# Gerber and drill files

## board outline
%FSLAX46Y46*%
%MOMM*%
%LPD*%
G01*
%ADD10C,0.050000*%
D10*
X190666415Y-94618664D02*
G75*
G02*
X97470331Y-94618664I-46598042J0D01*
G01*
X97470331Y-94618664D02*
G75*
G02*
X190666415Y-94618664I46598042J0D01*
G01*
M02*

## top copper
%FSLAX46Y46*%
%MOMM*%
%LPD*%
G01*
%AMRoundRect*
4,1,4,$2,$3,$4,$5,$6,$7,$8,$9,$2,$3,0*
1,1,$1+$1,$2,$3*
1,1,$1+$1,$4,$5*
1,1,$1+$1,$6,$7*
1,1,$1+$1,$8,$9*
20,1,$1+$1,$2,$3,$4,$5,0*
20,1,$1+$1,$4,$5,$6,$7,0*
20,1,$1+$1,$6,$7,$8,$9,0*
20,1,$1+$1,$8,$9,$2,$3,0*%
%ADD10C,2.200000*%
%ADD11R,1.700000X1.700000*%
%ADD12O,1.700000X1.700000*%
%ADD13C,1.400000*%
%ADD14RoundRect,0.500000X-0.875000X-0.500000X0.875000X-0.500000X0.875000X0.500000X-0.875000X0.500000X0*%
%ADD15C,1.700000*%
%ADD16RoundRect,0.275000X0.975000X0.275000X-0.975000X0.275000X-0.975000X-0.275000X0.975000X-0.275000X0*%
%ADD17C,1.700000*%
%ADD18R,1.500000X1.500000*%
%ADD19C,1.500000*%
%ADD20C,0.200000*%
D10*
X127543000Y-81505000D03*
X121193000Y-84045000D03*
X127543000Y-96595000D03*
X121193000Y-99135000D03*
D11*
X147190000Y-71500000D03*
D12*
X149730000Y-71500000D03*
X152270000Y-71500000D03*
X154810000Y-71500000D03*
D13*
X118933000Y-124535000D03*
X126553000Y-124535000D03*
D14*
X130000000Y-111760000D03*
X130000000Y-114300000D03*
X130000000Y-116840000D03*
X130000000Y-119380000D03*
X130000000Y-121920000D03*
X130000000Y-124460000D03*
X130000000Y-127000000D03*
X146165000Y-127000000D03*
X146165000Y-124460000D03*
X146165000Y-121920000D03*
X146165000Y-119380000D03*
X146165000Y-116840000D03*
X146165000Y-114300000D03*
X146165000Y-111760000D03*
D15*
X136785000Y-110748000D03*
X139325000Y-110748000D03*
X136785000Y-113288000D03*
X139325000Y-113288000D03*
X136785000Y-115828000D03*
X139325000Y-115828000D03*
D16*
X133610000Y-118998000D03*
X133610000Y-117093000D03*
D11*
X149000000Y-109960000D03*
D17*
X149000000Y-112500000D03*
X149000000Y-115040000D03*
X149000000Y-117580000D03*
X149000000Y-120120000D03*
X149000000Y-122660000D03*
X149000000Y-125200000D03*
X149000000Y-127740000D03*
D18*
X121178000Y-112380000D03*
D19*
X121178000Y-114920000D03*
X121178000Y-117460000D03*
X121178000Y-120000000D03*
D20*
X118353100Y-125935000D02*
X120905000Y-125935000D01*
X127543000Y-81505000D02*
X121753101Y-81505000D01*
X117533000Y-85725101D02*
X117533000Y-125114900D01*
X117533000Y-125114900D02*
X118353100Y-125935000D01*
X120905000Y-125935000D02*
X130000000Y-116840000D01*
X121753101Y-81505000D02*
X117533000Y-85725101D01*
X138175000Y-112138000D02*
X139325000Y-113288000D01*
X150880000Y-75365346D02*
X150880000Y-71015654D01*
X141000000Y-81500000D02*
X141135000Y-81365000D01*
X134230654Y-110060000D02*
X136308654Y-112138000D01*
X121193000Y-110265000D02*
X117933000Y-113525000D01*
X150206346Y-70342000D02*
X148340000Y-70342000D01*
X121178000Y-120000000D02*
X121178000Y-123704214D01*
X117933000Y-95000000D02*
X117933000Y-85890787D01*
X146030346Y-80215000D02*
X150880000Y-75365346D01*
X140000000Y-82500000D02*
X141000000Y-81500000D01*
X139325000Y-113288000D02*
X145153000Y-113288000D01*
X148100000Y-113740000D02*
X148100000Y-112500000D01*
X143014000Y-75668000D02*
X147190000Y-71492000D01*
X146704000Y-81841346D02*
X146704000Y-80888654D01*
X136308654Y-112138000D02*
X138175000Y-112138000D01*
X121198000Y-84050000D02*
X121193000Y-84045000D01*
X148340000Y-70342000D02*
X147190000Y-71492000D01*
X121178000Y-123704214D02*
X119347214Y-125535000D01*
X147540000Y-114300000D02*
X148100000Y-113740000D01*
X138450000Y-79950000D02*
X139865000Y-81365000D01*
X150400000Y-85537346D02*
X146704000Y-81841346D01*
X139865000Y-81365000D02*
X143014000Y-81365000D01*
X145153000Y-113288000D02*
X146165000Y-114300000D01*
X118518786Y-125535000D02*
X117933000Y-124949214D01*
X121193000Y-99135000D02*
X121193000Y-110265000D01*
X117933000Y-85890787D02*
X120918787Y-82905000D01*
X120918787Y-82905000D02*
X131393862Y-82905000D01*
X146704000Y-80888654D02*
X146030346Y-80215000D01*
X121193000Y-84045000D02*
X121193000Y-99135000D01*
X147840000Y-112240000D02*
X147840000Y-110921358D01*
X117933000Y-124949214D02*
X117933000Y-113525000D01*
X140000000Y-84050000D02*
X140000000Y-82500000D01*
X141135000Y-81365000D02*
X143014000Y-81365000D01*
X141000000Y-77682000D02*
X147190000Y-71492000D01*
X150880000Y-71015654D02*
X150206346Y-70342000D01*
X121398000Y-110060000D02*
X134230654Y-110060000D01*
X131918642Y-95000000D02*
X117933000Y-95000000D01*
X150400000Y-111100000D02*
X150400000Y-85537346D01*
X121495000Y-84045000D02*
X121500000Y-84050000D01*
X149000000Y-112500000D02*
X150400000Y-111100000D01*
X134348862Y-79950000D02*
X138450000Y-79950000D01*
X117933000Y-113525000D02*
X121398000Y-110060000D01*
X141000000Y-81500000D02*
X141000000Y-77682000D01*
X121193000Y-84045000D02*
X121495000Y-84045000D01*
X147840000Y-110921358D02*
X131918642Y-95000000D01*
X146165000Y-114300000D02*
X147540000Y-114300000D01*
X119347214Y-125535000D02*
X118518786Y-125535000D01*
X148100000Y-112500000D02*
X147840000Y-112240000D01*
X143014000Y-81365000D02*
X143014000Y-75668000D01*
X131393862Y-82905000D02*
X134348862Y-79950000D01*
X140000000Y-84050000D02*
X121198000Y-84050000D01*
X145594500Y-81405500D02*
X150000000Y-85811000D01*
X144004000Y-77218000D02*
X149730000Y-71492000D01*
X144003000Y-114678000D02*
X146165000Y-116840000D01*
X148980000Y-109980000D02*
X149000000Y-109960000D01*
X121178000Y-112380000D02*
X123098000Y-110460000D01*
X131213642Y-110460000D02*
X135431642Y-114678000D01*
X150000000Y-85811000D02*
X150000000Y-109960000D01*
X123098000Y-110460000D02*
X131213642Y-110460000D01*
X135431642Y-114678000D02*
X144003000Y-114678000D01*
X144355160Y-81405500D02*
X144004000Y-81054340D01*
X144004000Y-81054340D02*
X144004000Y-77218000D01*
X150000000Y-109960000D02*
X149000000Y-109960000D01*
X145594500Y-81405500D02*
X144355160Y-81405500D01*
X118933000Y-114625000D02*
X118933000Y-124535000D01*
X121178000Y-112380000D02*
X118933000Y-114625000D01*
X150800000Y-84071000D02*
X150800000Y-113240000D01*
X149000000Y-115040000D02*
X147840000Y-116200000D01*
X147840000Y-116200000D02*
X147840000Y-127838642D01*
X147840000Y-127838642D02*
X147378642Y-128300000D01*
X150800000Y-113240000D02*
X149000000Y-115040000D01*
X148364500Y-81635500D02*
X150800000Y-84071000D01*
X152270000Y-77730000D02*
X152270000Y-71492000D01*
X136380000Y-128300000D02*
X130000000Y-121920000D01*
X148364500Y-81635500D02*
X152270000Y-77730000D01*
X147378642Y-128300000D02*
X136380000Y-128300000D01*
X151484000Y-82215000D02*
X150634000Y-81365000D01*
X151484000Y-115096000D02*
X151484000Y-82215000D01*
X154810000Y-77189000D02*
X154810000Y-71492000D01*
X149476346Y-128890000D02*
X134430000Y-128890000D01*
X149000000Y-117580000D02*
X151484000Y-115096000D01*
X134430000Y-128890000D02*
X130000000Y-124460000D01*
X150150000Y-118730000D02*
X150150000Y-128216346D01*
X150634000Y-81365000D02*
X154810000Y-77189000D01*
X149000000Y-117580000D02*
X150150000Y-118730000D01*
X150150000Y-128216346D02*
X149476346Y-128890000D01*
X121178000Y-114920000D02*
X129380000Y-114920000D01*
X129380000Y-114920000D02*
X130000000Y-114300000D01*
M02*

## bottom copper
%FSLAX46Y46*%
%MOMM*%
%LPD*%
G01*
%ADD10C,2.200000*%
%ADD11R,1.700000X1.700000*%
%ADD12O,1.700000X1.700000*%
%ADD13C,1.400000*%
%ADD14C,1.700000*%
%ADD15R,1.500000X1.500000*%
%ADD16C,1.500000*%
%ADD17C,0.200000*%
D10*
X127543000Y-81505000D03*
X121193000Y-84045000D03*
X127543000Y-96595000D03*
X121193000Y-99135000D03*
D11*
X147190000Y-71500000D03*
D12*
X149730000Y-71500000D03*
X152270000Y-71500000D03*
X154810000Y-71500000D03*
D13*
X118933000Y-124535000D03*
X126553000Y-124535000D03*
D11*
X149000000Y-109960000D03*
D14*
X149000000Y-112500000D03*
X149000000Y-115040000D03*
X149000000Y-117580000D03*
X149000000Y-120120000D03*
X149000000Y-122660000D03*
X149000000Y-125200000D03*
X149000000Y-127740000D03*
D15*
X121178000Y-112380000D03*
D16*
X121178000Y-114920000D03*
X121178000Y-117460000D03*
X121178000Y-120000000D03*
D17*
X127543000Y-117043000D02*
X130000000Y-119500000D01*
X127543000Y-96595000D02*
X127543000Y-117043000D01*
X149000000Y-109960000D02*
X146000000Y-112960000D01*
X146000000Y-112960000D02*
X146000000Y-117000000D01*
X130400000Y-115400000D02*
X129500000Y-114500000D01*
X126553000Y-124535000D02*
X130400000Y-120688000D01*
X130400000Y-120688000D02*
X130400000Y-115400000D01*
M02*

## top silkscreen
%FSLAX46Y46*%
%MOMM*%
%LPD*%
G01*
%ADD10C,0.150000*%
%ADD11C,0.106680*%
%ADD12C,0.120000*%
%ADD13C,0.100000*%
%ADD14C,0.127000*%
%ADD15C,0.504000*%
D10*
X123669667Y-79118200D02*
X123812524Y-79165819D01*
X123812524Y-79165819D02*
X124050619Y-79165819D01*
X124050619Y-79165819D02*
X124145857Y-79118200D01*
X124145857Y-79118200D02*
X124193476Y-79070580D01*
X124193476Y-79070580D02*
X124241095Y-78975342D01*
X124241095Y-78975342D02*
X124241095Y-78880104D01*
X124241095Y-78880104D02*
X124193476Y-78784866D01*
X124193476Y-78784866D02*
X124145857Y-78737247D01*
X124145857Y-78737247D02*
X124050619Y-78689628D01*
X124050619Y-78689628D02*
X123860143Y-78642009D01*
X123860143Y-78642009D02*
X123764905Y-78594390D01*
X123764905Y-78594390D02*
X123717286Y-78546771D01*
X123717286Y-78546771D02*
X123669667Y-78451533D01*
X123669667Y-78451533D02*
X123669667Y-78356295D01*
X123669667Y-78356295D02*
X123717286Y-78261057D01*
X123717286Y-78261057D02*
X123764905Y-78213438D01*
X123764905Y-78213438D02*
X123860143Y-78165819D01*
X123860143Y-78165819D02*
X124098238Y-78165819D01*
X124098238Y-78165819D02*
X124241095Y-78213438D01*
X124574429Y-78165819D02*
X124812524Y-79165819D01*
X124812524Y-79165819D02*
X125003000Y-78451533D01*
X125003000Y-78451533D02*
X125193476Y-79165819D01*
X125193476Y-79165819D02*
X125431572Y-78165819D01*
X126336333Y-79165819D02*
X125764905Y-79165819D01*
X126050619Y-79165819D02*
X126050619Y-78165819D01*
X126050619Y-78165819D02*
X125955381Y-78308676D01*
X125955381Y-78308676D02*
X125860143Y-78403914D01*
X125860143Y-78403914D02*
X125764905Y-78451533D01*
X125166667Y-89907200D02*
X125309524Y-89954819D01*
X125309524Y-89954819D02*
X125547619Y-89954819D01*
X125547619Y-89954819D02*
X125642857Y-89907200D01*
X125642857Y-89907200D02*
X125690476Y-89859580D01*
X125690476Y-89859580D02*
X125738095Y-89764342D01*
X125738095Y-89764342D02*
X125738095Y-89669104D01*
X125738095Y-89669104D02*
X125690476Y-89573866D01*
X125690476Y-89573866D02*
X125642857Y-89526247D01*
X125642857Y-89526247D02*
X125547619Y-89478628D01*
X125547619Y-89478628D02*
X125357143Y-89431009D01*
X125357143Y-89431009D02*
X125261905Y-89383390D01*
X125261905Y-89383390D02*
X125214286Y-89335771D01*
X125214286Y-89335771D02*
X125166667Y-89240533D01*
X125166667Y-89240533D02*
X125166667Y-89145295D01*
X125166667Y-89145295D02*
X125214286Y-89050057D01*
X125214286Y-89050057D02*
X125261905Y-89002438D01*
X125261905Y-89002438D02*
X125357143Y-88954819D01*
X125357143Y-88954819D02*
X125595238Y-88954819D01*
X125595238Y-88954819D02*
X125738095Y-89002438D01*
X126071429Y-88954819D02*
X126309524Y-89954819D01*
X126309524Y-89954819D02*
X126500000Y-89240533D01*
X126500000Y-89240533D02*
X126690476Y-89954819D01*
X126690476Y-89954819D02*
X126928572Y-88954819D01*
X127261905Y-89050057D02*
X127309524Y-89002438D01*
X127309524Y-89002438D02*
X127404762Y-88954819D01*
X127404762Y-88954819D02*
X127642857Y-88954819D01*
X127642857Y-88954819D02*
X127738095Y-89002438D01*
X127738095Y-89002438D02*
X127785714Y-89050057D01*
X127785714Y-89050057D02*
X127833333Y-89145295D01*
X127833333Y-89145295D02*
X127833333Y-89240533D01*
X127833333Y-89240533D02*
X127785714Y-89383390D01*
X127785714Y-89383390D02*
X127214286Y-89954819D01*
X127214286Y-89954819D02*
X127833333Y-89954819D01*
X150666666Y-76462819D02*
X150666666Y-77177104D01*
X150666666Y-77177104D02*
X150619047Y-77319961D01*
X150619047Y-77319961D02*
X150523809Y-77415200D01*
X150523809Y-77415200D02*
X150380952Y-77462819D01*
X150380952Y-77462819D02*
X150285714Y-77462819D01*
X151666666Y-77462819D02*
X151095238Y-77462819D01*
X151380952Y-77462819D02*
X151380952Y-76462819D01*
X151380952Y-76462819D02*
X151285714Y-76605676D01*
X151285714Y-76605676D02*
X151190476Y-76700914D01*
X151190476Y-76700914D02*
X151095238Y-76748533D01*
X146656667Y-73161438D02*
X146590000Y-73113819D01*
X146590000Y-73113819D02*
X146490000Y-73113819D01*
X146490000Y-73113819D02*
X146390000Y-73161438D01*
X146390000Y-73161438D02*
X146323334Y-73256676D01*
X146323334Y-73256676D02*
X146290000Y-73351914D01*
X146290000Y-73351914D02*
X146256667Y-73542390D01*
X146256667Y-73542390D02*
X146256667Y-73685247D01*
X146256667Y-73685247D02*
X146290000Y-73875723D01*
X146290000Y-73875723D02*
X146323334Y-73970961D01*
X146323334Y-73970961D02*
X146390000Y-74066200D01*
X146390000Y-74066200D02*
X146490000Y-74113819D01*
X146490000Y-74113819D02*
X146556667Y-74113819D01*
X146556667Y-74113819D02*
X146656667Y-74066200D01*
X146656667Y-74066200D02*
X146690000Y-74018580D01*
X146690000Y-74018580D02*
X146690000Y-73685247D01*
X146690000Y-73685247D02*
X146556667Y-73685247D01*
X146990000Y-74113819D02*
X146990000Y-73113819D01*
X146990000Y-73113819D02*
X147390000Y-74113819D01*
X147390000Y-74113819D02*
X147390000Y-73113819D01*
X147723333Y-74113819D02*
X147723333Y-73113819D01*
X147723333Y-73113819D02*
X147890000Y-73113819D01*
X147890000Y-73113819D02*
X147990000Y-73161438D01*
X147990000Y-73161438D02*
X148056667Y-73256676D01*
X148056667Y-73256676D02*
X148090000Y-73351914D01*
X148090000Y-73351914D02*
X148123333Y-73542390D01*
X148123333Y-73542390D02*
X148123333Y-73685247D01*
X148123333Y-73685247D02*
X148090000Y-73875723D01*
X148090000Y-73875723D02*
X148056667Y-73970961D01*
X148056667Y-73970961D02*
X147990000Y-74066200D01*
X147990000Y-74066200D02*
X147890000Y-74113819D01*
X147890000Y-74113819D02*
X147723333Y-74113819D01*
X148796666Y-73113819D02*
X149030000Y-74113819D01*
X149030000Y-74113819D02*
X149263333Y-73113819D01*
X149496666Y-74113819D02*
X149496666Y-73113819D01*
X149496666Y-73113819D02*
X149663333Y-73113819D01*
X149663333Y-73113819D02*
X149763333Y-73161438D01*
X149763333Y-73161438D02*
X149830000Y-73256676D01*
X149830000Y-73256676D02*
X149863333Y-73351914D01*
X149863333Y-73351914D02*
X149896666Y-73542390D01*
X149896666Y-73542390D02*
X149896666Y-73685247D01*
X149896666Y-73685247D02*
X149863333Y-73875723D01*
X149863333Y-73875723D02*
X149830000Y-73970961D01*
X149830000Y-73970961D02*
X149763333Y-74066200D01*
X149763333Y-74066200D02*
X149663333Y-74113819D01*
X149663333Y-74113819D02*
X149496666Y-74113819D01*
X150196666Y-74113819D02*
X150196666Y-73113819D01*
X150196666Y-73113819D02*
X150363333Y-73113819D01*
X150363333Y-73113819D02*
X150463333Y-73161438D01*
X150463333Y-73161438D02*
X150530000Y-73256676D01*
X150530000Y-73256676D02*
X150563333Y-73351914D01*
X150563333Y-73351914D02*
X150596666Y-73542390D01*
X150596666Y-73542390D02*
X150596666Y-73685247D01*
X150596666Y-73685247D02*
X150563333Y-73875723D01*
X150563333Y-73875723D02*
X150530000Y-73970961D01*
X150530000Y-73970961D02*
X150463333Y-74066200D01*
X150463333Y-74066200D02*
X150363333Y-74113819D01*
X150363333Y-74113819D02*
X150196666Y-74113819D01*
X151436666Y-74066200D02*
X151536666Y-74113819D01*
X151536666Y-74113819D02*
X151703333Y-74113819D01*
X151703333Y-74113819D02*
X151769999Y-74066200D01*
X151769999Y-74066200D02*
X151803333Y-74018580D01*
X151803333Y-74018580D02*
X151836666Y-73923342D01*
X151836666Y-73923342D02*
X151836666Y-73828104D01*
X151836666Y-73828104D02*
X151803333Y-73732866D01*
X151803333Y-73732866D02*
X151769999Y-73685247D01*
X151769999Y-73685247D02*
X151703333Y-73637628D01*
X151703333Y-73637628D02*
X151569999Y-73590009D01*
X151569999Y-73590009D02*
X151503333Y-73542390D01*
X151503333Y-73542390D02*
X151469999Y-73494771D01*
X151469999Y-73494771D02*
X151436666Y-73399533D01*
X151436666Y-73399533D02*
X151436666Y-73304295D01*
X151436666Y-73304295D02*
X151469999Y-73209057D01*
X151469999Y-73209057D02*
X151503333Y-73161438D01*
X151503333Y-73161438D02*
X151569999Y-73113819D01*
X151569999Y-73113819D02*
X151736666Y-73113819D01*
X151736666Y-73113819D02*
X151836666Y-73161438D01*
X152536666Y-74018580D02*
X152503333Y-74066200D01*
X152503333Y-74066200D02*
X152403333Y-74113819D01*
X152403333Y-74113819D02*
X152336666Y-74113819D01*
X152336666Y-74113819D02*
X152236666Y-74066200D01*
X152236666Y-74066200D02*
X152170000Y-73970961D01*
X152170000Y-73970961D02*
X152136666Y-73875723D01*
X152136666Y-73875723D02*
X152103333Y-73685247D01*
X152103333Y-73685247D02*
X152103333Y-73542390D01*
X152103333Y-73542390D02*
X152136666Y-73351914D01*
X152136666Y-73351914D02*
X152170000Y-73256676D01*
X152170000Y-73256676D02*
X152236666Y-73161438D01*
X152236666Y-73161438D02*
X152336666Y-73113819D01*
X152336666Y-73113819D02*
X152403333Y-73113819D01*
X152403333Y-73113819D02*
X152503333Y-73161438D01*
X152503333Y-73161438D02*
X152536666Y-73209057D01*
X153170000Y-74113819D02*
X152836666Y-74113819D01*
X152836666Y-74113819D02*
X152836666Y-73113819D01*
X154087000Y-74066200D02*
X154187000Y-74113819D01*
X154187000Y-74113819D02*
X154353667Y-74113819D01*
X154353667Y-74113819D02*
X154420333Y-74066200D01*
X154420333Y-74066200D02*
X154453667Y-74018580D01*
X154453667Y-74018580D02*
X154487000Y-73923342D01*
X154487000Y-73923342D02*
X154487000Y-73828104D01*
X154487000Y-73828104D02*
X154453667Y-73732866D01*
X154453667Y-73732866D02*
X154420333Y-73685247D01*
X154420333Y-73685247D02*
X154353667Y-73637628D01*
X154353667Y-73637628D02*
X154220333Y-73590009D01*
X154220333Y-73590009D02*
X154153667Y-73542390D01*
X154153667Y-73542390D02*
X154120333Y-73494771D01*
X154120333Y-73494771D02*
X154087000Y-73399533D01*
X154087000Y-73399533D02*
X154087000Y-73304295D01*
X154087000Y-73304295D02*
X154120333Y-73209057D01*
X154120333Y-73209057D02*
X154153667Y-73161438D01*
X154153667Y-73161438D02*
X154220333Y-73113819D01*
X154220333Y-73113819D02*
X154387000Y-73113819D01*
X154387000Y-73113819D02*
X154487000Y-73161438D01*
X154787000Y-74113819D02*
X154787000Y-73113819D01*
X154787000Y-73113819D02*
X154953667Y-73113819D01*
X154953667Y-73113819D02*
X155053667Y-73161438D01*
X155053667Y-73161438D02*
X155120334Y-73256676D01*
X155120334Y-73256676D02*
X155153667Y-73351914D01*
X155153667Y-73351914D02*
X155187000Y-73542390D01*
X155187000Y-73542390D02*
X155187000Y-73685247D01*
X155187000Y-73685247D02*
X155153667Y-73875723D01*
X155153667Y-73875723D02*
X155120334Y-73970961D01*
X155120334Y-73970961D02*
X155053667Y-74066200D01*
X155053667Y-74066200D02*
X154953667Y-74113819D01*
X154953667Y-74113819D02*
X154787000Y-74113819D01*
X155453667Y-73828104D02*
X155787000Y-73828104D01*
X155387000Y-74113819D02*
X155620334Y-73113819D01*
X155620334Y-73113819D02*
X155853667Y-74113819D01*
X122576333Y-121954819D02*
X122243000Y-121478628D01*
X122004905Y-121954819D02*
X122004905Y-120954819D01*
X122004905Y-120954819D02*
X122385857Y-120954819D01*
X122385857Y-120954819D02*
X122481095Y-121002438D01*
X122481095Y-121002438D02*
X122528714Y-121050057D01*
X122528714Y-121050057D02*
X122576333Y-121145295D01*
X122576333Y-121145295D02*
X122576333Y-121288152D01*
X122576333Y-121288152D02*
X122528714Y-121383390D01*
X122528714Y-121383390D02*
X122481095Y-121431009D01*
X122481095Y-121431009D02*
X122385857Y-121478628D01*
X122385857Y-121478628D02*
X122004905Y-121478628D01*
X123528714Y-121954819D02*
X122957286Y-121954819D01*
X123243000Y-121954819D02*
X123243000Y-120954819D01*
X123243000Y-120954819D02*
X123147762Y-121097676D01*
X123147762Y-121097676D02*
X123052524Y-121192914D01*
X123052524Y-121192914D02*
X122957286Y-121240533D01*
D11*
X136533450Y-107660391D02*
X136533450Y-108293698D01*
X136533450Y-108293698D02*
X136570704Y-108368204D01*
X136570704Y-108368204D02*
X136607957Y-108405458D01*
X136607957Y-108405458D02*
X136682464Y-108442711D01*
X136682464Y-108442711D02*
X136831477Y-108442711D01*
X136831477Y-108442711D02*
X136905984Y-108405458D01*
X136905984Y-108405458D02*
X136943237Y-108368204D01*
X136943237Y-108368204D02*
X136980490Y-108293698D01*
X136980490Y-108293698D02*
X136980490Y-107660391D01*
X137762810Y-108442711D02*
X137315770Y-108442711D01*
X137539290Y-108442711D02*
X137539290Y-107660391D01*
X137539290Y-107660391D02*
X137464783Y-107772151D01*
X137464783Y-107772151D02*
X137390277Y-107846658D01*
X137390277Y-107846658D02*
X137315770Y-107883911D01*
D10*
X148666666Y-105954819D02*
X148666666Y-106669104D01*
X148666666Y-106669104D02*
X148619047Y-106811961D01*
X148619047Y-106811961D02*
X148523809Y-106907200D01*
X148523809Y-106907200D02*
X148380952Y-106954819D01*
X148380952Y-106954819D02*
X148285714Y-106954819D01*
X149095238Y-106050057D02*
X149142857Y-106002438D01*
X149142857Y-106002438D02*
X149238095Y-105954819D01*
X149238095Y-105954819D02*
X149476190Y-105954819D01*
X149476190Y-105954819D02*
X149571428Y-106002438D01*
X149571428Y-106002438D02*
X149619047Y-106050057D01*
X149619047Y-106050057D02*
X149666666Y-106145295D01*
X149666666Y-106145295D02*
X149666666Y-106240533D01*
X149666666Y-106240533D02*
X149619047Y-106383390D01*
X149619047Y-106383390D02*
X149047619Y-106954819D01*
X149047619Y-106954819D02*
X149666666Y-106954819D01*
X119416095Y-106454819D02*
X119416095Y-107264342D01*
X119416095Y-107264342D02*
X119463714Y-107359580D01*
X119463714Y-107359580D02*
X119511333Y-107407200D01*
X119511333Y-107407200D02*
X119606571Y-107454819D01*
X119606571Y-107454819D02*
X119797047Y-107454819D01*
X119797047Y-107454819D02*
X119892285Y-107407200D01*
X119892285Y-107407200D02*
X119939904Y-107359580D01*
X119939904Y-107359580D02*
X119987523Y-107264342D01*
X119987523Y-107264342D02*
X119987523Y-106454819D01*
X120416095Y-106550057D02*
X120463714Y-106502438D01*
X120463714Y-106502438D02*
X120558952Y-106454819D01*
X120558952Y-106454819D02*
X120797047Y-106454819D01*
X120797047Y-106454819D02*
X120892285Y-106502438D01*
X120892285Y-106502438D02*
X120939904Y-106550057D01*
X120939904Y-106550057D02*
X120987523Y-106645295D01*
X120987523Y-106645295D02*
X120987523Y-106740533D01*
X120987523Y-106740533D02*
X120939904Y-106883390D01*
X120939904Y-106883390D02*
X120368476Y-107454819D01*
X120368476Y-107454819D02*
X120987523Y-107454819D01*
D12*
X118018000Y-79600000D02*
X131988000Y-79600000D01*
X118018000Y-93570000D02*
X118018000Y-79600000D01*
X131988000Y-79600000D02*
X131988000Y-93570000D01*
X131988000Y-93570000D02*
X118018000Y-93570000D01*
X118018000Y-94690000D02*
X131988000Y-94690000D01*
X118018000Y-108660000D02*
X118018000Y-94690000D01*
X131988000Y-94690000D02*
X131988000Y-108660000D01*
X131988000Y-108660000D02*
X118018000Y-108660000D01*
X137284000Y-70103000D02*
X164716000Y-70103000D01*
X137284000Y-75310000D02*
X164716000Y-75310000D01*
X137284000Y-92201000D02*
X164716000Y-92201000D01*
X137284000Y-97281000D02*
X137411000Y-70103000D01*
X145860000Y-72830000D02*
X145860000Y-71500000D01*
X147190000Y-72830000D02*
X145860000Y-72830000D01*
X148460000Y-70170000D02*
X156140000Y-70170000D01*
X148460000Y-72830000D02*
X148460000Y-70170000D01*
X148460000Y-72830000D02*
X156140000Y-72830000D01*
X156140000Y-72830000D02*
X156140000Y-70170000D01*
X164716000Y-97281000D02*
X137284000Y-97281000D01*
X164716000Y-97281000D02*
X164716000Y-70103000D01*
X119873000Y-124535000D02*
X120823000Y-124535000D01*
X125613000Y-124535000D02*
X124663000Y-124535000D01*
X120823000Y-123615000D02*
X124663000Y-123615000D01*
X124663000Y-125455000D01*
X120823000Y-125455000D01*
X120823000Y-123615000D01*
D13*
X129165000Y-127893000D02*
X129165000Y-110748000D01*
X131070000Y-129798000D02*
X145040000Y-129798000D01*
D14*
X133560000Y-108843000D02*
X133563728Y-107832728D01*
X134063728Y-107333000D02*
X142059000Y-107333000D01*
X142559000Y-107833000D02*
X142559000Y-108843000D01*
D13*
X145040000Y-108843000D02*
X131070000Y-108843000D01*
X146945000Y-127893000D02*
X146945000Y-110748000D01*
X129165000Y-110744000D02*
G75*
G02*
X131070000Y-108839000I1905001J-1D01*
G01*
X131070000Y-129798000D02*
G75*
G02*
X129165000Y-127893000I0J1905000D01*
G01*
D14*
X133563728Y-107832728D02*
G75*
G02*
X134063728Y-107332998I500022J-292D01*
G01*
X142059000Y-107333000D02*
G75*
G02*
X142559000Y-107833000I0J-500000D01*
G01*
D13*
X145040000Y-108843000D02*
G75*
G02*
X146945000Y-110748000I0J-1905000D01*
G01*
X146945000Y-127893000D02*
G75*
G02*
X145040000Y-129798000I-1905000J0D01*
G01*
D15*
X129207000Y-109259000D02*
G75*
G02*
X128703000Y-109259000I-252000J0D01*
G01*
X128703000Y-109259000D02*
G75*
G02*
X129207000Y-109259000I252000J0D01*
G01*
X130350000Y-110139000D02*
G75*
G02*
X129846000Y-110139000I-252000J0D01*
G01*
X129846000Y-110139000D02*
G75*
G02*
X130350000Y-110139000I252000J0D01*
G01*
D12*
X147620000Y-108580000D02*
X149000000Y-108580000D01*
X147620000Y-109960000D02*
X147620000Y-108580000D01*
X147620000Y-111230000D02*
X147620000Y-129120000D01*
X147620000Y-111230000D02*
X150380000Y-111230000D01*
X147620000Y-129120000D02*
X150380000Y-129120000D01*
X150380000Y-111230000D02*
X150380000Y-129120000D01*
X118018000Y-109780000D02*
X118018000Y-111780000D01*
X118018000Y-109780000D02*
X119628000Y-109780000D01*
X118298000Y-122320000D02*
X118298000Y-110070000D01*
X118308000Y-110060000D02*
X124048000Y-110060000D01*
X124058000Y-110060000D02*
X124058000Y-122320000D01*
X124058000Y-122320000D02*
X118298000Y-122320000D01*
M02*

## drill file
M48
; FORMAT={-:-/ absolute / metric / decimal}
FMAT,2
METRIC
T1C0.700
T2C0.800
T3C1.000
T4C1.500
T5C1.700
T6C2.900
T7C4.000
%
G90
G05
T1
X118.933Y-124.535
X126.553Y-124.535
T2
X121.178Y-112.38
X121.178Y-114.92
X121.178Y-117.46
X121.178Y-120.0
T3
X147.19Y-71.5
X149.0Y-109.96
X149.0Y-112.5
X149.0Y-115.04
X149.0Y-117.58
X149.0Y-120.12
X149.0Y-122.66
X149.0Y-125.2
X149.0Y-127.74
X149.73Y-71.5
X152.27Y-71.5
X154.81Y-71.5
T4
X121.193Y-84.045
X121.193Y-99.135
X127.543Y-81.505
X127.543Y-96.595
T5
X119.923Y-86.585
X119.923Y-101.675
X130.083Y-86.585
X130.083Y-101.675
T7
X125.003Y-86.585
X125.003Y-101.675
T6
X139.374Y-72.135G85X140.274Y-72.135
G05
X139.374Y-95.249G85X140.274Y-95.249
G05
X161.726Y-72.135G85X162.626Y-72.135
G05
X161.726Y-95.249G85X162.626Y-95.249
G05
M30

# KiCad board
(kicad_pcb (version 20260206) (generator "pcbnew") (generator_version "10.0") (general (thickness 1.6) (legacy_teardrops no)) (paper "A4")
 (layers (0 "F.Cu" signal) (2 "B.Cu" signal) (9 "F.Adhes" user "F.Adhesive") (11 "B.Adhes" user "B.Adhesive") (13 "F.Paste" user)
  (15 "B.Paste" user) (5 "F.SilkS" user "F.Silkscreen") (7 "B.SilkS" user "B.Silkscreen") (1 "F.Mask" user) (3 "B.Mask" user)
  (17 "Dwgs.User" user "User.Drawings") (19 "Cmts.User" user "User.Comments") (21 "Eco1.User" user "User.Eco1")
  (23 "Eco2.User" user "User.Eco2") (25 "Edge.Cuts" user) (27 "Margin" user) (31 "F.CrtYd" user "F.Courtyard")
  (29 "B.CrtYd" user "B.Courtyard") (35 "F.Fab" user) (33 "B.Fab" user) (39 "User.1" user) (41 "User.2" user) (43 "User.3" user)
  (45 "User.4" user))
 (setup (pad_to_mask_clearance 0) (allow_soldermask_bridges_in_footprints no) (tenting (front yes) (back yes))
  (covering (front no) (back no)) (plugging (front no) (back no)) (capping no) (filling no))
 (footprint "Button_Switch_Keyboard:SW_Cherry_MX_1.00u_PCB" (layer "F.Cu") (at 127.543 81.505)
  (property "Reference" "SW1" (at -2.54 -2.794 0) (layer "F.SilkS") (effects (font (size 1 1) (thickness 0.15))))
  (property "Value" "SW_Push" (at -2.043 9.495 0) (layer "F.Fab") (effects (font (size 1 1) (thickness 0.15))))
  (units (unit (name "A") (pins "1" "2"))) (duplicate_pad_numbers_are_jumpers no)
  (fp_line (start -9.525 -1.905) (end 4.445 -1.905) (stroke (width 0.12) (type solid)) (layer "F.SilkS"))
  (fp_line (start -9.525 12.065) (end -9.525 -1.905) (stroke (width 0.12) (type solid)) (layer "F.SilkS"))
  (fp_line (start 4.445 -1.905) (end 4.445 12.065) (stroke (width 0.12) (type solid)) (layer "F.SilkS"))
  (fp_line (start 4.445 12.065) (end -9.525 12.065) (stroke (width 0.12) (type solid)) (layer "F.SilkS"))
  (pad "" np_thru_hole circle (at -7.62 5.08) (size 1.7 1.7) (drill 1.7) (layers "*.Cu" "*.Mask"))
  (pad "" np_thru_hole circle (at -2.54 5.08) (size 4 4) (drill 4) (layers "*.Cu" "*.Mask"))
  (pad "" np_thru_hole circle (at 2.54 5.08) (size 1.7 1.7) (drill 1.7) (layers "*.Cu" "*.Mask"))
  (pad "1" thru_hole circle (at 0 0) (size 2.2 2.2) (drill 1.5) (layers "*.Cu" "*.Mask") (remove_unused_layers no) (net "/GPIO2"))
  (pad "2" thru_hole circle (at -6.35 2.54) (size 2.2 2.2) (drill 1.5) (layers "*.Cu" "*.Mask") (remove_unused_layers no) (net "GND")))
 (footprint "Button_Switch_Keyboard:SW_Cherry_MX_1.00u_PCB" (layer "F.Cu") (at 127.543 96.595)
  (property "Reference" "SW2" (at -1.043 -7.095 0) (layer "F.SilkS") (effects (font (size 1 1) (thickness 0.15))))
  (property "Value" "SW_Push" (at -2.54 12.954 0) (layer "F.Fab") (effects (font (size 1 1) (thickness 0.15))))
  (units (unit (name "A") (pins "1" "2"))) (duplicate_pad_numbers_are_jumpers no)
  (fp_line (start -9.525 -1.905) (end 4.445 -1.905) (stroke (width 0.12) (type solid)) (layer "F.SilkS"))
  (fp_line (start -9.525 12.065) (end -9.525 -1.905) (stroke (width 0.12) (type solid)) (layer "F.SilkS"))
  (fp_line (start 4.445 -1.905) (end 4.445 12.065) (stroke (width 0.12) (type solid)) (layer "F.SilkS"))
  (fp_line (start 4.445 12.065) (end -9.525 12.065) (stroke (width 0.12) (type solid)) (layer "F.SilkS"))
  (pad "" np_thru_hole circle (at -7.62 5.08) (size 1.7 1.7) (drill 1.7) (layers "*.Cu" "*.Mask"))
  (pad "" np_thru_hole circle (at -2.54 5.08) (size 4 4) (drill 4) (layers "*.Cu" "*.Mask"))
  (pad "" np_thru_hole circle (at 2.54 5.08) (size 1.7 1.7) (drill 1.7) (layers "*.Cu" "*.Mask"))
  (pad "1" thru_hole circle (at 0 0) (size 2.2 2.2) (drill 1.5) (layers "*.Cu" "*.Mask") (remove_unused_layers no) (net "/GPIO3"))
  (pad "2" thru_hole circle (at -6.35 2.54) (size 2.2 2.2) (drill 1.5) (layers "*.Cu" "*.Mask") (remove_unused_layers no) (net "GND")))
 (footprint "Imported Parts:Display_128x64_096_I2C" (layer "F.Cu") (at 151 71.5)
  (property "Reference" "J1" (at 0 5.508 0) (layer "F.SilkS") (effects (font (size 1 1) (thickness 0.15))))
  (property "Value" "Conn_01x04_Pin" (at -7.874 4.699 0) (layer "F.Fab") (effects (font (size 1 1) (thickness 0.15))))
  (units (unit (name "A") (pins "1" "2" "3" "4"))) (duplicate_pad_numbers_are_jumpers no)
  (fp_line (start -13.716 -1.397) (end 13.716 -1.397) (stroke (width 0.12) (type solid)) (layer "F.SilkS"))
  (fp_line (start -13.716 3.81) (end 13.716 3.81) (stroke (width 0.12) (type solid)) (layer "F.SilkS"))
  (fp_line (start -13.716 20.701) (end 13.716 20.701) (stroke (width 0.12) (type solid)) (layer "F.SilkS"))
  (fp_line (start -13.716 25.781) (end -13.589 -1.397) (stroke (width 0.12) (type solid)) (layer "F.SilkS"))
  (fp_line (start -5.14 1.33) (end -5.14 0) (stroke (width 0.12) (type solid)) (layer "F.SilkS"))
  (fp_line (start -3.81 1.33) (end -5.14 1.33) (stroke (width 0.12) (type solid)) (layer "F.SilkS"))
  (fp_line (start -2.54 -1.33) (end 5.14 -1.33) (stroke (width 0.12) (type solid)) (layer "F.SilkS"))
  (fp_line (start -2.54 1.33) (end -2.54 -1.33) (stroke (width 0.12) (type solid)) (layer "F.SilkS"))
  (fp_line (start -2.54 1.33) (end 5.14 1.33) (stroke (width 0.12) (type solid)) (layer "F.SilkS"))
  (fp_line (start 5.14 1.33) (end 5.14 -1.33) (stroke (width 0.12) (type solid)) (layer "F.SilkS"))
  (fp_line (start 13.716 25.781) (end -13.716 25.781) (stroke (width 0.12) (type solid)) (layer "F.SilkS"))
  (fp_line (start 13.716 25.781) (end 13.716 -1.397) (stroke (width 0.12) (type solid)) (layer "F.SilkS"))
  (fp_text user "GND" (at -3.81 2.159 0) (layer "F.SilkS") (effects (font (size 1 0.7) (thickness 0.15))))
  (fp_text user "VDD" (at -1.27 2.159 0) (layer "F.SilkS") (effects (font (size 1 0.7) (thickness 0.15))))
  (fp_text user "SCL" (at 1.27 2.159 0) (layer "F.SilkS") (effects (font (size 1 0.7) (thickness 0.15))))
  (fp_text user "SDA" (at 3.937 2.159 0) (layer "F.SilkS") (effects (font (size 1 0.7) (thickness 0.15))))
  (pad "" np_thru_hole oval (at -11.176 0.635) (size 3.8 2.9) (drill oval 3.8 2.9) (layers "*.Cu" "*.Mask"))
  (pad "" np_thru_hole oval (at -11.176 23.749) (size 3.8 2.9) (drill oval 3.8 2.9) (layers "*.Cu" "*.Mask"))
  (pad "" np_thru_hole oval (at 11.176 0.635) (size 3.8 2.9) (drill oval 3.8 2.9) (layers "*.Cu" "*.Mask"))
  (pad "" np_thru_hole oval (at 11.176 23.749) (size 3.8 2.9) (drill oval 3.8 2.9) (layers "*.Cu" "*.Mask"))
  (pad "1" thru_hole rect (at -3.81 0 90) (size 1.7 1.7) (drill 1) (layers "*.Cu" "*.Mask") (remove_unused_layers no) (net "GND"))
  (pad "2" thru_hole oval (at -1.27 0 90) (size 1.7 1.7) (drill 1) (layers "*.Cu" "*.Mask") (remove_unused_layers no) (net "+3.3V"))
  (pad "3" thru_hole oval (at 1.27 0 90) (size 1.7 1.7) (drill 1) (layers "*.Cu" "*.Mask") (remove_unused_layers no) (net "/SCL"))
  (pad "4" thru_hole oval (at 3.81 0 90) (size 1.7 1.7) (drill 1) (layers "*.Cu" "*.Mask") (remove_unused_layers no) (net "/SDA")))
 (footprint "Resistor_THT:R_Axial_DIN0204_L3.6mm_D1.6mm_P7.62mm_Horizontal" (layer "F.Cu") (at 118.933 124.535)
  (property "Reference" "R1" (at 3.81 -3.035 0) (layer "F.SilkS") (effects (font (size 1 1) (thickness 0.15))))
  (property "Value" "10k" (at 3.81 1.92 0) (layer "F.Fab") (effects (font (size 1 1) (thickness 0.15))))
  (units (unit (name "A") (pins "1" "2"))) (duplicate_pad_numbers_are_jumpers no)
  (fp_line (start 0.94 0) (end 1.89 0) (stroke (width 0.12) (type solid)) (layer "F.SilkS"))
  (fp_line (start 6.68 0) (end 5.73 0) (stroke (width 0.12) (type solid)) (layer "F.SilkS"))
  (fp_rect (start 1.89 -0.92) (end 5.73 0.92) (stroke (width 0.12) (type solid)) (fill no) (layer "F.SilkS"))
  (pad "1" thru_hole circle (at 0 0) (size 1.4 1.4) (drill 0.7) (layers "*.Cu" "*.Mask") (remove_unused_layers no) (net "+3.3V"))
  (pad "2" thru_hole circle (at 7.62 0) (size 1.4 1.4) (drill 0.7) (layers "*.Cu" "*.Mask") (remove_unused_layers no) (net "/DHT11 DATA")))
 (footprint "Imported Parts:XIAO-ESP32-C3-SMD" (layer "F.Cu") (at 129.165 129.88)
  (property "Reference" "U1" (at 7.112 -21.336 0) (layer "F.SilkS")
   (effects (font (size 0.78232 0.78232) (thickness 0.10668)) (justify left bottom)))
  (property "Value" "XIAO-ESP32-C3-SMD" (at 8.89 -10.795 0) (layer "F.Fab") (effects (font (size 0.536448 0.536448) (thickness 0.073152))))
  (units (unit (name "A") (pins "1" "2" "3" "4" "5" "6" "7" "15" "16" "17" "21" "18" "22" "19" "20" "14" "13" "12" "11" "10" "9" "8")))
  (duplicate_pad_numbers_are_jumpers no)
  (fp_line (start 0 -1.987) (end 0 -19.132) (stroke (width 0.1) (type solid)) (layer "F.SilkS"))
  (fp_line (start 1.905 -0.082) (end 15.875 -0.082) (stroke (width 0.1) (type solid)) (layer "F.SilkS"))
  (fp_line (start 4.395 -21.037) (end 4.398728 -22.047272) (stroke (width 0.127) (type solid)) (layer "F.SilkS"))
  (fp_line (start 4.898728 -22.547) (end 12.894 -22.547) (stroke (width 0.127) (type solid)) (layer "F.SilkS"))
  (fp_line (start 13.394 -22.047) (end 13.394 -21.037) (stroke (width 0.127) (type solid)) (layer "F.SilkS"))
  (fp_line (start 15.875 -21.037) (end 1.905 -21.037) (stroke (width 0.1) (type solid)) (layer "F.SilkS"))
  (fp_line (start 17.78 -1.987) (end 17.78 -19.132) (stroke (width 0.1) (type solid)) (layer "F.SilkS"))
  (fp_arc (start 0 -19.136) (mid 0.557962 -20.483038) (end 1.905 -21.041) (stroke (width 0.1) (type solid)) (layer "F.SilkS"))
  (fp_arc (start 1.905 -0.082) (mid 0.557962 -0.639962) (end 0 -1.987) (stroke (width 0.1) (type solid)) (layer "F.SilkS"))
  (fp_arc (start 4.398728 -22.047272) (mid 4.545272 -22.40064) (end 4.898728 -22.547) (stroke (width 0.127) (type default))
   (layer "F.SilkS"))
  (fp_arc (start 12.894 -22.547) (mid 13.247553 -22.400553) (end 13.394 -22.047) (stroke (width 0.127) (type default)) (layer "F.SilkS"))
  (fp_arc (start 15.875 -21.037) (mid 17.222038 -20.479038) (end 17.78 -19.132) (stroke (width 0.1) (type solid)) (layer "F.SilkS"))
  (fp_arc (start 17.78 -1.987) (mid 17.222038 -0.639962) (end 15.875 -0.082) (stroke (width 0.1) (type solid)) (layer "F.SilkS"))
  (fp_circle (center -0.21 -20.621) (end -0.21 -20.875) (stroke (width 0.5) (type solid)) (fill yes) (layer "F.SilkS"))
  (fp_circle (center 0.933 -19.741) (end 0.933 -19.995) (stroke (width 0.5) (type solid)) (fill yes) (layer "F.SilkS"))
  (pad "1" smd roundrect (at 0.835 -18.12) (size 2.75 2) (layers "F.Cu" "F.Mask" "F.Paste") (roundrect_rratio 0.25)
   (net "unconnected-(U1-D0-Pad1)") (solder_mask_margin 0.0508) (thermal_bridge_angle 45))
  (pad "2" smd roundrect (at 0.835 -15.58) (size 2.75 2) (layers "F.Cu" "F.Mask" "F.Paste") (roundrect_rratio 0.25) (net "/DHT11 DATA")
   (solder_mask_margin 0.0508) (thermal_bridge_angle 45))
  (pad "3" smd roundrect (at 0.835 -13.04) (size 2.75 2) (layers "F.Cu" "F.Mask" "F.Paste") (roundrect_rratio 0.25) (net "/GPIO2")
   (solder_mask_margin 0.0508) (thermal_bridge_angle 45))
  (pad "4" smd roundrect (at 0.835 -10.5) (size 2.75 2) (layers "F.Cu" "F.Mask" "F.Paste") (roundrect_rratio 0.25) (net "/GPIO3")
   (solder_mask_margin 0.0508) (thermal_bridge_angle 45))
  (pad "5" smd roundrect (at 0.835 -7.96) (size 2.75 2) (layers "F.Cu" "F.Mask" "F.Paste") (roundrect_rratio 0.25) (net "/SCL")
   (solder_mask_margin 0.0508) (thermal_bridge_angle 45))
  (pad "6" smd roundrect (at 0.835 -5.42) (size 2.75 2) (layers "F.Cu" "F.Mask" "F.Paste") (roundrect_rratio 0.25) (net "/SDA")
   (solder_mask_margin 0.0508) (thermal_bridge_angle 45))
  (pad "7" smd roundrect (at 0.835 -2.88) (size 2.75 2) (layers "F.Cu" "F.Mask" "F.Paste") (roundrect_rratio 0.25)
   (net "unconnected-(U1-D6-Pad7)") (solder_mask_margin 0.0508) (thermal_bridge_angle 45))
  (pad "8" smd roundrect (at 17 -2.88) (size 2.75 2) (layers "F.Cu" "F.Mask" "F.Paste") (roundrect_rratio 0.25)
   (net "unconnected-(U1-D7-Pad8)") (solder_mask_margin 0.0508) (thermal_bridge_angle 45))
  (pad "9" smd roundrect (at 17 -5.42) (size 2.75 2) (layers "F.Cu" "F.Mask" "F.Paste") (roundrect_rratio 0.25)
   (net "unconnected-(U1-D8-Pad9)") (solder_mask_margin 0.0508) (thermal_bridge_angle 45))
  (pad "10" smd roundrect (at 17 -7.96) (size 2.75 2) (layers "F.Cu" "F.Mask" "F.Paste") (roundrect_rratio 0.25)
   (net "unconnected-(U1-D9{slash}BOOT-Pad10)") (solder_mask_margin 0.0508) (thermal_bridge_angle 45))
  (pad "11" smd roundrect (at 17 -10.5) (size 2.75 2) (layers "F.Cu" "F.Mask" "F.Paste") (roundrect_rratio 0.25)
   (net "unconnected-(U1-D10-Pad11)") (solder_mask_margin 0.0508) (thermal_bridge_angle 45))
  (pad "12" smd roundrect (at 17 -13.04) (size 2.75 2) (layers "F.Cu" "F.Mask" "F.Paste") (roundrect_rratio 0.25) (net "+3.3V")
   (solder_mask_margin 0.0508) (thermal_bridge_angle 45))
  (pad "13" smd roundrect (at 17 -15.58) (size 2.75 2) (layers "F.Cu" "F.Mask" "F.Paste") (roundrect_rratio 0.25) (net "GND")
   (solder_mask_margin 0.0508) (thermal_bridge_angle 45))
  (pad "14" smd roundrect (at 17 -18.12) (size 2.75 2) (layers "F.Cu" "F.Mask" "F.Paste") (roundrect_rratio 0.25) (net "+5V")
   (solder_mask_margin 0.0508) (thermal_bridge_angle 45))
  (pad "15" smd circle (at 7.62 -19.132) (size 1.7 1.7) (layers "F.Cu" "F.Mask" "F.Paste") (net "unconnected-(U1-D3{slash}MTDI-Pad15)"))
  (pad "16" smd circle (at 10.16 -19.132) (size 1.7 1.7) (layers "F.Cu" "F.Mask" "F.Paste") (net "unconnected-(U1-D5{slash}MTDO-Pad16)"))
  (pad "17" smd circle (at 7.62 -16.592) (size 1.7 1.7) (layers "F.Cu" "F.Mask" "F.Paste") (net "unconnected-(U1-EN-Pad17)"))
  (pad "18" smd circle (at 10.16 -16.592) (size 1.7 1.7) (layers "F.Cu" "F.Mask" "F.Paste") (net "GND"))
  (pad "19" smd circle (at 7.62 -14.052) (size 1.7 1.7) (layers "F.Cu" "F.Mask" "F.Paste") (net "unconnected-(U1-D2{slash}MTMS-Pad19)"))
  (pad "20" smd circle (at 10.16 -14.052) (size 1.7 1.7) (layers "F.Cu" "F.Mask" "F.Paste") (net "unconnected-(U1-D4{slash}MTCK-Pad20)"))
  (pad "21" smd roundrect (at 4.445 -10.882 180) (size 2.5 1.1) (layers "F.Cu" "F.Mask" "F.Paste") (roundrect_rratio 0.25)
   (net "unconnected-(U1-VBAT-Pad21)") (thermal_bridge_angle 45))
  (pad "22" smd roundrect (at 4.445 -12.787 180) (size 2.5 1.1) (layers "F.Cu" "F.Mask" "F.Paste") (roundrect_rratio 0.25)
   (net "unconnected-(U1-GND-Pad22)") (thermal_bridge_angle 45)))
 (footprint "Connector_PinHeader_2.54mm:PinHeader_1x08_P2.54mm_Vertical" (layer "F.Cu") (at 149 109.96)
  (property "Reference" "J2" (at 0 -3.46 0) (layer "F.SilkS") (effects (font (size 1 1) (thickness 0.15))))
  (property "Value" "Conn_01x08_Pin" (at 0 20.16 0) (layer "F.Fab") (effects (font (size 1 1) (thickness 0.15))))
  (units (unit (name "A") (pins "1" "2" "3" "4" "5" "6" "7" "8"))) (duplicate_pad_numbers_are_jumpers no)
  (fp_line (start -1.38 -1.38) (end 0 -1.38) (stroke (width 0.12) (type solid)) (layer "F.SilkS"))
  (fp_line (start -1.38 0) (end -1.38 -1.38) (stroke (width 0.12) (type solid)) (layer "F.SilkS"))
  (fp_line (start -1.38 1.27) (end -1.38 19.16) (stroke (width 0.12) (type solid)) (layer "F.SilkS"))
  (fp_line (start -1.38 1.27) (end 1.38 1.27) (stroke (width 0.12) (type solid)) (layer "F.SilkS"))
  (fp_line (start -1.38 19.16) (end 1.38 19.16) (stroke (width 0.12) (type solid)) (layer "F.SilkS"))
  (fp_line (start 1.38 1.27) (end 1.38 19.16) (stroke (width 0.12) (type solid)) (layer "F.SilkS"))
  (pad "1" thru_hole rect (at 0 0) (size 1.7 1.7) (drill 1) (layers "*.Cu" "*.Mask") (remove_unused_layers no) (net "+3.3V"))
  (pad "2" thru_hole circle (at 0 2.54) (size 1.7 1.7) (drill 1) (layers "*.Cu" "*.Mask") (remove_unused_layers no) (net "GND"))
  (pad "3" thru_hole circle (at 0 5.08) (size 1.7 1.7) (drill 1) (layers "*.Cu" "*.Mask") (remove_unused_layers no) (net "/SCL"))
  (pad "4" thru_hole circle (at 0 7.62) (size 1.7 1.7) (drill 1) (layers "*.Cu" "*.Mask") (remove_unused_layers no) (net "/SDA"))
  (pad "5" thru_hole circle (at 0 10.16) (size 1.7 1.7) (drill 1) (layers "*.Cu" "*.Mask") (remove_unused_layers no)
   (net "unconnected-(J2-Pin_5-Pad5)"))
  (pad "6" thru_hole circle (at 0 12.7) (size 1.7 1.7) (drill 1) (layers "*.Cu" "*.Mask") (remove_unused_layers no)
   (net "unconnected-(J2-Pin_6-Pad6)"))
  (pad "7" thru_hole circle (at 0 15.24) (size 1.7 1.7) (drill 1) (layers "*.Cu" "*.Mask") (remove_unused_layers no)
   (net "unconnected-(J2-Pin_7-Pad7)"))
  (pad "8" thru_hole circle (at 0 17.78) (size 1.7 1.7) (drill 1) (layers "*.Cu" "*.Mask") (remove_unused_layers no)
   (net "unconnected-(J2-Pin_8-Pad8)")))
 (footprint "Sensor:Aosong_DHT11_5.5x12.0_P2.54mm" (layer "F.Cu") (at 121.178 112.38)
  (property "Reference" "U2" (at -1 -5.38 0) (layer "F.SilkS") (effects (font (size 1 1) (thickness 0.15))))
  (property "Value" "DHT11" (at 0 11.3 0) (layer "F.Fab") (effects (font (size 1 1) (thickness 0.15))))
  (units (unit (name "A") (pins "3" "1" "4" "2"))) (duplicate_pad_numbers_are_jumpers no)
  (fp_line (start -3.16 -2.6) (end -3.16 -0.6) (stroke (width 0.12) (type solid)) (layer "F.SilkS"))
  (fp_line (start -3.16 -2.6) (end -1.55 -2.6) (stroke (width 0.12) (type solid)) (layer "F.SilkS"))
  (fp_line (start -2.88 9.94) (end -2.88 -2.31) (stroke (width 0.12) (type solid)) (layer "F.SilkS"))
  (fp_line (start -2.87 -2.32) (end 2.87 -2.32) (stroke (width 0.12) (type solid)) (layer "F.SilkS"))
  (fp_line (start 2.88 -2.32) (end 2.88 9.94) (stroke (width 0.12) (type solid)) (layer "F.SilkS"))
  (fp_line (start 2.88 9.94) (end -2.88 9.94) (stroke (width 0.12) (type solid)) (layer "F.SilkS"))
  (pad "1" thru_hole rect (at 0 0) (size 1.5 1.5) (drill 0.8) (layers "*.Cu" "*.Mask") (remove_unused_layers no) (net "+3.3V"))
  (pad "2" thru_hole circle (at 0 2.54) (size 1.5 1.5) (drill 0.8) (layers "*.Cu" "*.Mask") (remove_unused_layers no) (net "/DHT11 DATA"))
  (pad "3" thru_hole circle (at 0 5.08) (size 1.5 1.5) (drill 0.8) (layers "*.Cu" "*.Mask") (remove_unused_layers no)
   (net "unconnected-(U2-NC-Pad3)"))
  (pad "4" thru_hole circle (at 0 7.62) (size 1.5 1.5) (drill 0.8) (layers "*.Cu" "*.Mask") (remove_unused_layers no) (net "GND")))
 (gr_circle (center 144.068373 94.618664) (end 107.5 123.5) (stroke (width 0.05) (type default)) (fill no) (layer "Edge.Cuts"))
 (segment (start 118.3531 125.935) (end 120.905 125.935) (width 0.2) (layer "F.Cu") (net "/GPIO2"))
 (segment (start 127.543 81.505) (end 121.753101 81.505) (width 0.2) (layer "F.Cu") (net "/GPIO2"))
 (segment (start 117.533 85.725101) (end 117.533 125.1149) (width 0.2) (layer "F.Cu") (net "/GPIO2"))
 (segment (start 117.533 125.1149) (end 118.3531 125.935) (width 0.2) (layer "F.Cu") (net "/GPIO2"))
 (segment (start 120.905 125.935) (end 130 116.84) (width 0.2) (layer "F.Cu") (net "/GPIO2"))
 (segment (start 121.753101 81.505) (end 117.533 85.725101) (width 0.2) (layer "F.Cu") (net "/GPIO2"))
 (segment (start 138.175 112.138) (end 139.325 113.288) (width 0.2) (layer "F.Cu") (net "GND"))
 (segment (start 150.88 75.365346) (end 150.88 71.015654) (width 0.2) (layer "F.Cu") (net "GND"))
 (segment (start 141 81.5) (end 141.135 81.365) (width 0.2) (layer "F.Cu") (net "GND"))
 (segment (start 134.230654 110.06) (end 136.308654 112.138) (width 0.2) (layer "F.Cu") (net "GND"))
 (segment (start 121.193 110.265) (end 117.933 113.525) (width 0.2) (layer "F.Cu") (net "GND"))
 (segment (start 150.206346 70.342) (end 148.34 70.342) (width 0.2) (layer "F.Cu") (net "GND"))
 (segment (start 121.178 120) (end 121.178 123.704214) (width 0.2) (layer "F.Cu") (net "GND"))
 (segment (start 117.933 95) (end 117.933 85.890787) (width 0.2) (layer "F.Cu") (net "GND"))
 (segment (start 146.030346 80.215) (end 150.88 75.365346) (width 0.2) (layer "F.Cu") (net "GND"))
 (segment (start 140 82.5) (end 141 81.5) (width 0.2) (layer "F.Cu") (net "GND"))
 (segment (start 139.325 113.288) (end 145.153 113.288) (width 0.2) (layer "F.Cu") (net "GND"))
 (segment (start 148.1 113.74) (end 148.1 112.5) (width 0.2) (layer "F.Cu") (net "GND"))
 (segment (start 143.014 75.668) (end 147.19 71.492) (width 0.2) (layer "F.Cu") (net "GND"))
 (segment (start 146.704 81.841346) (end 146.704 80.888654) (width 0.2) (layer "F.Cu") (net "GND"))
 (segment (start 136.308654 112.138) (end 138.175 112.138) (width 0.2) (layer "F.Cu") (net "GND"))
 (segment (start 121.198 84.05) (end 121.193 84.045) (width 0.2) (layer "F.Cu") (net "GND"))
 (segment (start 148.34 70.342) (end 147.19 71.492) (width 0.2) (layer "F.Cu") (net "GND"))
 (segment (start 121.178 123.704214) (end 119.347214 125.535) (width 0.2) (layer "F.Cu") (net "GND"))
 (segment (start 147.54 114.3) (end 148.1 113.74) (width 0.2) (layer "F.Cu") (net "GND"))
 (segment (start 138.45 79.95) (end 139.865 81.365) (width 0.2) (layer "F.Cu") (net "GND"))
 (segment (start 150.4 85.537346) (end 146.704 81.841346) (width 0.2) (layer "F.Cu") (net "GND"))
 (segment (start 139.865 81.365) (end 143.014 81.365) (width 0.2) (layer "F.Cu") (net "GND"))
 (segment (start 145.153 113.288) (end 146.165 114.3) (width 0.2) (layer "F.Cu") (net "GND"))
 (segment (start 118.518786 125.535) (end 117.933 124.949214) (width 0.2) (layer "F.Cu") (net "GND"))
 (segment (start 121.193 99.135) (end 121.193 110.265) (width 0.2) (layer "F.Cu") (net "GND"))
 (segment (start 117.933 85.890787) (end 120.918787 82.905) (width 0.2) (layer "F.Cu") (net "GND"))
 (segment (start 120.918787 82.905) (end 131.393862 82.905) (width 0.2) (layer "F.Cu") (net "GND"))
 (segment (start 146.704 80.888654) (end 146.030346 80.215) (width 0.2) (layer "F.Cu") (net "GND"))
 (segment (start 121.193 84.045) (end 121.193 99.135) (width 0.2) (layer "F.Cu") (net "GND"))
 (segment (start 147.84 112.24) (end 147.84 110.921358) (width 0.2) (layer "F.Cu") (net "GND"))
 (segment (start 117.933 124.949214) (end 117.933 113.525) (width 0.2) (layer "F.Cu") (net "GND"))
 (segment (start 140 84.05) (end 140 82.5) (width 0.2) (layer "F.Cu") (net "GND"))
 (segment (start 141.135 81.365) (end 143.014 81.365) (width 0.2) (layer "F.Cu") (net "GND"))
 (segment (start 141 77.682) (end 147.19 71.492) (width 0.2) (layer "F.Cu") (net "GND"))
 (segment (start 150.88 71.015654) (end 150.206346 70.342) (width 0.2) (layer "F.Cu") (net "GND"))
 (segment (start 121.398 110.06) (end 134.230654 110.06) (width 0.2) (layer "F.Cu") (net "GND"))
 (segment (start 131.918642 95) (end 117.933 95) (width 0.2) (layer "F.Cu") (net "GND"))
 (segment (start 150.4 111.1) (end 150.4 85.537346) (width 0.2) (layer "F.Cu") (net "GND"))
 (segment (start 121.495 84.045) (end 121.5 84.05) (width 0.2) (layer "F.Cu") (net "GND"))
 (segment (start 149 112.5) (end 150.4 111.1) (width 0.2) (layer "F.Cu") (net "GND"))
 (segment (start 134.348862 79.95) (end 138.45 79.95) (width 0.2) (layer "F.Cu") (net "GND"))
 (segment (start 117.933 113.525) (end 121.398 110.06) (width 0.2) (layer "F.Cu") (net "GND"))
 (segment (start 141 81.5) (end 141 77.682) (width 0.2) (layer "F.Cu") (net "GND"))
 (segment (start 121.193 84.045) (end 121.495 84.045) (width 0.2) (layer "F.Cu") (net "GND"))
 (segment (start 147.84 110.921358) (end 131.918642 95) (width 0.2) (layer "F.Cu") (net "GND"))
 (segment (start 146.165 114.3) (end 147.54 114.3) (width 0.2) (layer "F.Cu") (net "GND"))
 (segment (start 119.347214 125.535) (end 118.518786 125.535) (width 0.2) (layer "F.Cu") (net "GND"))
 (segment (start 148.1 112.5) (end 147.84 112.24) (width 0.2) (layer "F.Cu") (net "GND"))
 (segment (start 143.014 81.365) (end 143.014 75.668) (width 0.2) (layer "F.Cu") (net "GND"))
 (segment (start 131.393862 82.905) (end 134.348862 79.95) (width 0.2) (layer "F.Cu") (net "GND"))
 (segment (start 140 84.05) (end 121.198 84.05) (width 0.2) (layer "F.Cu") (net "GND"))
 (segment (start 127.543 117.043) (end 130 119.5) (width 0.2) (layer "B.Cu") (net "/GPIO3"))
 (segment (start 127.543 96.595) (end 127.543 117.043) (width 0.2) (layer "B.Cu") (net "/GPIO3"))
 (segment (start 145.5945 81.4055) (end 150 85.811) (width 0.2) (layer "F.Cu") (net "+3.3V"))
 (segment (start 144.004 77.218) (end 149.73 71.492) (width 0.2) (layer "F.Cu") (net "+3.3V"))
 (segment (start 144.003 114.678) (end 146.165 116.84) (width 0.2) (layer "F.Cu") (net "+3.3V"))
 (segment (start 148.98 109.98) (end 149 109.96) (width 0.2) (layer "F.Cu") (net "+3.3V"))
 (segment (start 121.178 112.38) (end 123.098 110.46) (width 0.2) (layer "F.Cu") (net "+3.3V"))
 (segment (start 131.213642 110.46) (end 135.431642 114.678) (width 0.2) (layer "F.Cu") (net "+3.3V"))
 (segment (start 150 85.811) (end 150 109.96) (width 0.2) (layer "F.Cu") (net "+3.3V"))
 (segment (start 123.098 110.46) (end 131.213642 110.46) (width 0.2) (layer "F.Cu") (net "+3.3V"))
 (segment (start 135.431642 114.678) (end 144.003 114.678) (width 0.2) (layer "F.Cu") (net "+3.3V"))
 (segment (start 144.35516 81.4055) (end 144.004 81.05434) (width 0.2) (layer "F.Cu") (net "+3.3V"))
 (segment (start 144.004 81.05434) (end 144.004 77.218) (width 0.2) (layer "F.Cu") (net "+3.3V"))
 (segment (start 150 109.96) (end 149 109.96) (width 0.2) (layer "F.Cu") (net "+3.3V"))
 (segment (start 145.5945 81.4055) (end 144.35516 81.4055) (width 0.2) (layer "F.Cu") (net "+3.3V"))
 (segment (start 118.933 114.625) (end 118.933 124.535) (width 0.2) (layer "F.Cu") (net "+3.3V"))
 (segment (start 121.178 112.38) (end 118.933 114.625) (width 0.2) (layer "F.Cu") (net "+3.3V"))
 (segment (start 149 109.96) (end 146 112.96) (width 0.2) (layer "B.Cu") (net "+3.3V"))
 (segment (start 146 112.96) (end 146 117) (width 0.2) (layer "B.Cu") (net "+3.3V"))
 (segment (start 150.8 84.071) (end 150.8 113.24) (width 0.2) (layer "F.Cu") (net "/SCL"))
 (segment (start 149 115.04) (end 147.84 116.2) (width 0.2) (layer "F.Cu") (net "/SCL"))
 (segment (start 147.84 116.2) (end 147.84 127.838642) (width 0.2) (layer "F.Cu") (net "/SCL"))
 (segment (start 147.84 127.838642) (end 147.378642 128.3) (width 0.2) (layer "F.Cu") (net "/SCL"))
 (segment (start 150.8 113.24) (end 149 115.04) (width 0.2) (layer "F.Cu") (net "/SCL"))
 (segment (start 148.3645 81.6355) (end 150.8 84.071) (width 0.2) (layer "F.Cu") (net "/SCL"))
 (segment (start 152.27 77.73) (end 152.27 71.492) (width 0.2) (layer "F.Cu") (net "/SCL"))
 (segment (start 136.38 128.3) (end 130 121.92) (width 0.2) (layer "F.Cu") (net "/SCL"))
 (segment (start 148.3645 81.6355) (end 152.27 77.73) (width 0.2) (layer "F.Cu") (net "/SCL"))
 (segment (start 147.378642 128.3) (end 136.38 128.3) (width 0.2) (layer "F.Cu") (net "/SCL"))
 (segment (start 151.484 82.215) (end 150.634 81.365) (width 0.2) (layer "F.Cu") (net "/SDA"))
 (segment (start 151.484 115.096) (end 151.484 82.215) (width 0.2) (layer "F.Cu") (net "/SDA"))
 (segment (start 154.81 77.189) (end 154.81 71.492) (width 0.2) (layer "F.Cu") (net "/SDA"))
 (segment (start 149.476346 128.89) (end 134.43 128.89) (width 0.2) (layer "F.Cu") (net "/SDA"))
 (segment (start 149 117.58) (end 151.484 115.096) (width 0.2) (layer "F.Cu") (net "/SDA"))
 (segment (start 134.43 128.89) (end 130 124.46) (width 0.2) (layer "F.Cu") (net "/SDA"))
 (segment (start 150.15 118.73) (end 150.15 128.216346) (width 0.2) (layer "F.Cu") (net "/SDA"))
 (segment (start 150.634 81.365) (end 154.81 77.189) (width 0.2) (layer "F.Cu") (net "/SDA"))
 (segment (start 149 117.58) (end 150.15 118.73) (width 0.2) (layer "F.Cu") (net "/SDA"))
 (segment (start 150.15 128.216346) (end 149.476346 128.89) (width 0.2) (layer "F.Cu") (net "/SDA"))
 (segment (start 121.178 114.92) (end 129.38 114.92) (width 0.2) (layer "F.Cu") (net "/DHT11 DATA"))
 (segment (start 129.38 114.92) (end 130 114.3) (width 0.2) (layer "F.Cu") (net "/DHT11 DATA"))
 (segment (start 130.4 115.4) (end 129.5 114.5) (width 0.2) (layer "B.Cu") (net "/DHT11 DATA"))
 (segment (start 126.553 124.535) (end 130.4 120.688) (width 0.2) (layer "B.Cu") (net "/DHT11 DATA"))
 (segment (start 130.4 120.688) (end 130.4 115.4) (width 0.2) (layer "B.Cu") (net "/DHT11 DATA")))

